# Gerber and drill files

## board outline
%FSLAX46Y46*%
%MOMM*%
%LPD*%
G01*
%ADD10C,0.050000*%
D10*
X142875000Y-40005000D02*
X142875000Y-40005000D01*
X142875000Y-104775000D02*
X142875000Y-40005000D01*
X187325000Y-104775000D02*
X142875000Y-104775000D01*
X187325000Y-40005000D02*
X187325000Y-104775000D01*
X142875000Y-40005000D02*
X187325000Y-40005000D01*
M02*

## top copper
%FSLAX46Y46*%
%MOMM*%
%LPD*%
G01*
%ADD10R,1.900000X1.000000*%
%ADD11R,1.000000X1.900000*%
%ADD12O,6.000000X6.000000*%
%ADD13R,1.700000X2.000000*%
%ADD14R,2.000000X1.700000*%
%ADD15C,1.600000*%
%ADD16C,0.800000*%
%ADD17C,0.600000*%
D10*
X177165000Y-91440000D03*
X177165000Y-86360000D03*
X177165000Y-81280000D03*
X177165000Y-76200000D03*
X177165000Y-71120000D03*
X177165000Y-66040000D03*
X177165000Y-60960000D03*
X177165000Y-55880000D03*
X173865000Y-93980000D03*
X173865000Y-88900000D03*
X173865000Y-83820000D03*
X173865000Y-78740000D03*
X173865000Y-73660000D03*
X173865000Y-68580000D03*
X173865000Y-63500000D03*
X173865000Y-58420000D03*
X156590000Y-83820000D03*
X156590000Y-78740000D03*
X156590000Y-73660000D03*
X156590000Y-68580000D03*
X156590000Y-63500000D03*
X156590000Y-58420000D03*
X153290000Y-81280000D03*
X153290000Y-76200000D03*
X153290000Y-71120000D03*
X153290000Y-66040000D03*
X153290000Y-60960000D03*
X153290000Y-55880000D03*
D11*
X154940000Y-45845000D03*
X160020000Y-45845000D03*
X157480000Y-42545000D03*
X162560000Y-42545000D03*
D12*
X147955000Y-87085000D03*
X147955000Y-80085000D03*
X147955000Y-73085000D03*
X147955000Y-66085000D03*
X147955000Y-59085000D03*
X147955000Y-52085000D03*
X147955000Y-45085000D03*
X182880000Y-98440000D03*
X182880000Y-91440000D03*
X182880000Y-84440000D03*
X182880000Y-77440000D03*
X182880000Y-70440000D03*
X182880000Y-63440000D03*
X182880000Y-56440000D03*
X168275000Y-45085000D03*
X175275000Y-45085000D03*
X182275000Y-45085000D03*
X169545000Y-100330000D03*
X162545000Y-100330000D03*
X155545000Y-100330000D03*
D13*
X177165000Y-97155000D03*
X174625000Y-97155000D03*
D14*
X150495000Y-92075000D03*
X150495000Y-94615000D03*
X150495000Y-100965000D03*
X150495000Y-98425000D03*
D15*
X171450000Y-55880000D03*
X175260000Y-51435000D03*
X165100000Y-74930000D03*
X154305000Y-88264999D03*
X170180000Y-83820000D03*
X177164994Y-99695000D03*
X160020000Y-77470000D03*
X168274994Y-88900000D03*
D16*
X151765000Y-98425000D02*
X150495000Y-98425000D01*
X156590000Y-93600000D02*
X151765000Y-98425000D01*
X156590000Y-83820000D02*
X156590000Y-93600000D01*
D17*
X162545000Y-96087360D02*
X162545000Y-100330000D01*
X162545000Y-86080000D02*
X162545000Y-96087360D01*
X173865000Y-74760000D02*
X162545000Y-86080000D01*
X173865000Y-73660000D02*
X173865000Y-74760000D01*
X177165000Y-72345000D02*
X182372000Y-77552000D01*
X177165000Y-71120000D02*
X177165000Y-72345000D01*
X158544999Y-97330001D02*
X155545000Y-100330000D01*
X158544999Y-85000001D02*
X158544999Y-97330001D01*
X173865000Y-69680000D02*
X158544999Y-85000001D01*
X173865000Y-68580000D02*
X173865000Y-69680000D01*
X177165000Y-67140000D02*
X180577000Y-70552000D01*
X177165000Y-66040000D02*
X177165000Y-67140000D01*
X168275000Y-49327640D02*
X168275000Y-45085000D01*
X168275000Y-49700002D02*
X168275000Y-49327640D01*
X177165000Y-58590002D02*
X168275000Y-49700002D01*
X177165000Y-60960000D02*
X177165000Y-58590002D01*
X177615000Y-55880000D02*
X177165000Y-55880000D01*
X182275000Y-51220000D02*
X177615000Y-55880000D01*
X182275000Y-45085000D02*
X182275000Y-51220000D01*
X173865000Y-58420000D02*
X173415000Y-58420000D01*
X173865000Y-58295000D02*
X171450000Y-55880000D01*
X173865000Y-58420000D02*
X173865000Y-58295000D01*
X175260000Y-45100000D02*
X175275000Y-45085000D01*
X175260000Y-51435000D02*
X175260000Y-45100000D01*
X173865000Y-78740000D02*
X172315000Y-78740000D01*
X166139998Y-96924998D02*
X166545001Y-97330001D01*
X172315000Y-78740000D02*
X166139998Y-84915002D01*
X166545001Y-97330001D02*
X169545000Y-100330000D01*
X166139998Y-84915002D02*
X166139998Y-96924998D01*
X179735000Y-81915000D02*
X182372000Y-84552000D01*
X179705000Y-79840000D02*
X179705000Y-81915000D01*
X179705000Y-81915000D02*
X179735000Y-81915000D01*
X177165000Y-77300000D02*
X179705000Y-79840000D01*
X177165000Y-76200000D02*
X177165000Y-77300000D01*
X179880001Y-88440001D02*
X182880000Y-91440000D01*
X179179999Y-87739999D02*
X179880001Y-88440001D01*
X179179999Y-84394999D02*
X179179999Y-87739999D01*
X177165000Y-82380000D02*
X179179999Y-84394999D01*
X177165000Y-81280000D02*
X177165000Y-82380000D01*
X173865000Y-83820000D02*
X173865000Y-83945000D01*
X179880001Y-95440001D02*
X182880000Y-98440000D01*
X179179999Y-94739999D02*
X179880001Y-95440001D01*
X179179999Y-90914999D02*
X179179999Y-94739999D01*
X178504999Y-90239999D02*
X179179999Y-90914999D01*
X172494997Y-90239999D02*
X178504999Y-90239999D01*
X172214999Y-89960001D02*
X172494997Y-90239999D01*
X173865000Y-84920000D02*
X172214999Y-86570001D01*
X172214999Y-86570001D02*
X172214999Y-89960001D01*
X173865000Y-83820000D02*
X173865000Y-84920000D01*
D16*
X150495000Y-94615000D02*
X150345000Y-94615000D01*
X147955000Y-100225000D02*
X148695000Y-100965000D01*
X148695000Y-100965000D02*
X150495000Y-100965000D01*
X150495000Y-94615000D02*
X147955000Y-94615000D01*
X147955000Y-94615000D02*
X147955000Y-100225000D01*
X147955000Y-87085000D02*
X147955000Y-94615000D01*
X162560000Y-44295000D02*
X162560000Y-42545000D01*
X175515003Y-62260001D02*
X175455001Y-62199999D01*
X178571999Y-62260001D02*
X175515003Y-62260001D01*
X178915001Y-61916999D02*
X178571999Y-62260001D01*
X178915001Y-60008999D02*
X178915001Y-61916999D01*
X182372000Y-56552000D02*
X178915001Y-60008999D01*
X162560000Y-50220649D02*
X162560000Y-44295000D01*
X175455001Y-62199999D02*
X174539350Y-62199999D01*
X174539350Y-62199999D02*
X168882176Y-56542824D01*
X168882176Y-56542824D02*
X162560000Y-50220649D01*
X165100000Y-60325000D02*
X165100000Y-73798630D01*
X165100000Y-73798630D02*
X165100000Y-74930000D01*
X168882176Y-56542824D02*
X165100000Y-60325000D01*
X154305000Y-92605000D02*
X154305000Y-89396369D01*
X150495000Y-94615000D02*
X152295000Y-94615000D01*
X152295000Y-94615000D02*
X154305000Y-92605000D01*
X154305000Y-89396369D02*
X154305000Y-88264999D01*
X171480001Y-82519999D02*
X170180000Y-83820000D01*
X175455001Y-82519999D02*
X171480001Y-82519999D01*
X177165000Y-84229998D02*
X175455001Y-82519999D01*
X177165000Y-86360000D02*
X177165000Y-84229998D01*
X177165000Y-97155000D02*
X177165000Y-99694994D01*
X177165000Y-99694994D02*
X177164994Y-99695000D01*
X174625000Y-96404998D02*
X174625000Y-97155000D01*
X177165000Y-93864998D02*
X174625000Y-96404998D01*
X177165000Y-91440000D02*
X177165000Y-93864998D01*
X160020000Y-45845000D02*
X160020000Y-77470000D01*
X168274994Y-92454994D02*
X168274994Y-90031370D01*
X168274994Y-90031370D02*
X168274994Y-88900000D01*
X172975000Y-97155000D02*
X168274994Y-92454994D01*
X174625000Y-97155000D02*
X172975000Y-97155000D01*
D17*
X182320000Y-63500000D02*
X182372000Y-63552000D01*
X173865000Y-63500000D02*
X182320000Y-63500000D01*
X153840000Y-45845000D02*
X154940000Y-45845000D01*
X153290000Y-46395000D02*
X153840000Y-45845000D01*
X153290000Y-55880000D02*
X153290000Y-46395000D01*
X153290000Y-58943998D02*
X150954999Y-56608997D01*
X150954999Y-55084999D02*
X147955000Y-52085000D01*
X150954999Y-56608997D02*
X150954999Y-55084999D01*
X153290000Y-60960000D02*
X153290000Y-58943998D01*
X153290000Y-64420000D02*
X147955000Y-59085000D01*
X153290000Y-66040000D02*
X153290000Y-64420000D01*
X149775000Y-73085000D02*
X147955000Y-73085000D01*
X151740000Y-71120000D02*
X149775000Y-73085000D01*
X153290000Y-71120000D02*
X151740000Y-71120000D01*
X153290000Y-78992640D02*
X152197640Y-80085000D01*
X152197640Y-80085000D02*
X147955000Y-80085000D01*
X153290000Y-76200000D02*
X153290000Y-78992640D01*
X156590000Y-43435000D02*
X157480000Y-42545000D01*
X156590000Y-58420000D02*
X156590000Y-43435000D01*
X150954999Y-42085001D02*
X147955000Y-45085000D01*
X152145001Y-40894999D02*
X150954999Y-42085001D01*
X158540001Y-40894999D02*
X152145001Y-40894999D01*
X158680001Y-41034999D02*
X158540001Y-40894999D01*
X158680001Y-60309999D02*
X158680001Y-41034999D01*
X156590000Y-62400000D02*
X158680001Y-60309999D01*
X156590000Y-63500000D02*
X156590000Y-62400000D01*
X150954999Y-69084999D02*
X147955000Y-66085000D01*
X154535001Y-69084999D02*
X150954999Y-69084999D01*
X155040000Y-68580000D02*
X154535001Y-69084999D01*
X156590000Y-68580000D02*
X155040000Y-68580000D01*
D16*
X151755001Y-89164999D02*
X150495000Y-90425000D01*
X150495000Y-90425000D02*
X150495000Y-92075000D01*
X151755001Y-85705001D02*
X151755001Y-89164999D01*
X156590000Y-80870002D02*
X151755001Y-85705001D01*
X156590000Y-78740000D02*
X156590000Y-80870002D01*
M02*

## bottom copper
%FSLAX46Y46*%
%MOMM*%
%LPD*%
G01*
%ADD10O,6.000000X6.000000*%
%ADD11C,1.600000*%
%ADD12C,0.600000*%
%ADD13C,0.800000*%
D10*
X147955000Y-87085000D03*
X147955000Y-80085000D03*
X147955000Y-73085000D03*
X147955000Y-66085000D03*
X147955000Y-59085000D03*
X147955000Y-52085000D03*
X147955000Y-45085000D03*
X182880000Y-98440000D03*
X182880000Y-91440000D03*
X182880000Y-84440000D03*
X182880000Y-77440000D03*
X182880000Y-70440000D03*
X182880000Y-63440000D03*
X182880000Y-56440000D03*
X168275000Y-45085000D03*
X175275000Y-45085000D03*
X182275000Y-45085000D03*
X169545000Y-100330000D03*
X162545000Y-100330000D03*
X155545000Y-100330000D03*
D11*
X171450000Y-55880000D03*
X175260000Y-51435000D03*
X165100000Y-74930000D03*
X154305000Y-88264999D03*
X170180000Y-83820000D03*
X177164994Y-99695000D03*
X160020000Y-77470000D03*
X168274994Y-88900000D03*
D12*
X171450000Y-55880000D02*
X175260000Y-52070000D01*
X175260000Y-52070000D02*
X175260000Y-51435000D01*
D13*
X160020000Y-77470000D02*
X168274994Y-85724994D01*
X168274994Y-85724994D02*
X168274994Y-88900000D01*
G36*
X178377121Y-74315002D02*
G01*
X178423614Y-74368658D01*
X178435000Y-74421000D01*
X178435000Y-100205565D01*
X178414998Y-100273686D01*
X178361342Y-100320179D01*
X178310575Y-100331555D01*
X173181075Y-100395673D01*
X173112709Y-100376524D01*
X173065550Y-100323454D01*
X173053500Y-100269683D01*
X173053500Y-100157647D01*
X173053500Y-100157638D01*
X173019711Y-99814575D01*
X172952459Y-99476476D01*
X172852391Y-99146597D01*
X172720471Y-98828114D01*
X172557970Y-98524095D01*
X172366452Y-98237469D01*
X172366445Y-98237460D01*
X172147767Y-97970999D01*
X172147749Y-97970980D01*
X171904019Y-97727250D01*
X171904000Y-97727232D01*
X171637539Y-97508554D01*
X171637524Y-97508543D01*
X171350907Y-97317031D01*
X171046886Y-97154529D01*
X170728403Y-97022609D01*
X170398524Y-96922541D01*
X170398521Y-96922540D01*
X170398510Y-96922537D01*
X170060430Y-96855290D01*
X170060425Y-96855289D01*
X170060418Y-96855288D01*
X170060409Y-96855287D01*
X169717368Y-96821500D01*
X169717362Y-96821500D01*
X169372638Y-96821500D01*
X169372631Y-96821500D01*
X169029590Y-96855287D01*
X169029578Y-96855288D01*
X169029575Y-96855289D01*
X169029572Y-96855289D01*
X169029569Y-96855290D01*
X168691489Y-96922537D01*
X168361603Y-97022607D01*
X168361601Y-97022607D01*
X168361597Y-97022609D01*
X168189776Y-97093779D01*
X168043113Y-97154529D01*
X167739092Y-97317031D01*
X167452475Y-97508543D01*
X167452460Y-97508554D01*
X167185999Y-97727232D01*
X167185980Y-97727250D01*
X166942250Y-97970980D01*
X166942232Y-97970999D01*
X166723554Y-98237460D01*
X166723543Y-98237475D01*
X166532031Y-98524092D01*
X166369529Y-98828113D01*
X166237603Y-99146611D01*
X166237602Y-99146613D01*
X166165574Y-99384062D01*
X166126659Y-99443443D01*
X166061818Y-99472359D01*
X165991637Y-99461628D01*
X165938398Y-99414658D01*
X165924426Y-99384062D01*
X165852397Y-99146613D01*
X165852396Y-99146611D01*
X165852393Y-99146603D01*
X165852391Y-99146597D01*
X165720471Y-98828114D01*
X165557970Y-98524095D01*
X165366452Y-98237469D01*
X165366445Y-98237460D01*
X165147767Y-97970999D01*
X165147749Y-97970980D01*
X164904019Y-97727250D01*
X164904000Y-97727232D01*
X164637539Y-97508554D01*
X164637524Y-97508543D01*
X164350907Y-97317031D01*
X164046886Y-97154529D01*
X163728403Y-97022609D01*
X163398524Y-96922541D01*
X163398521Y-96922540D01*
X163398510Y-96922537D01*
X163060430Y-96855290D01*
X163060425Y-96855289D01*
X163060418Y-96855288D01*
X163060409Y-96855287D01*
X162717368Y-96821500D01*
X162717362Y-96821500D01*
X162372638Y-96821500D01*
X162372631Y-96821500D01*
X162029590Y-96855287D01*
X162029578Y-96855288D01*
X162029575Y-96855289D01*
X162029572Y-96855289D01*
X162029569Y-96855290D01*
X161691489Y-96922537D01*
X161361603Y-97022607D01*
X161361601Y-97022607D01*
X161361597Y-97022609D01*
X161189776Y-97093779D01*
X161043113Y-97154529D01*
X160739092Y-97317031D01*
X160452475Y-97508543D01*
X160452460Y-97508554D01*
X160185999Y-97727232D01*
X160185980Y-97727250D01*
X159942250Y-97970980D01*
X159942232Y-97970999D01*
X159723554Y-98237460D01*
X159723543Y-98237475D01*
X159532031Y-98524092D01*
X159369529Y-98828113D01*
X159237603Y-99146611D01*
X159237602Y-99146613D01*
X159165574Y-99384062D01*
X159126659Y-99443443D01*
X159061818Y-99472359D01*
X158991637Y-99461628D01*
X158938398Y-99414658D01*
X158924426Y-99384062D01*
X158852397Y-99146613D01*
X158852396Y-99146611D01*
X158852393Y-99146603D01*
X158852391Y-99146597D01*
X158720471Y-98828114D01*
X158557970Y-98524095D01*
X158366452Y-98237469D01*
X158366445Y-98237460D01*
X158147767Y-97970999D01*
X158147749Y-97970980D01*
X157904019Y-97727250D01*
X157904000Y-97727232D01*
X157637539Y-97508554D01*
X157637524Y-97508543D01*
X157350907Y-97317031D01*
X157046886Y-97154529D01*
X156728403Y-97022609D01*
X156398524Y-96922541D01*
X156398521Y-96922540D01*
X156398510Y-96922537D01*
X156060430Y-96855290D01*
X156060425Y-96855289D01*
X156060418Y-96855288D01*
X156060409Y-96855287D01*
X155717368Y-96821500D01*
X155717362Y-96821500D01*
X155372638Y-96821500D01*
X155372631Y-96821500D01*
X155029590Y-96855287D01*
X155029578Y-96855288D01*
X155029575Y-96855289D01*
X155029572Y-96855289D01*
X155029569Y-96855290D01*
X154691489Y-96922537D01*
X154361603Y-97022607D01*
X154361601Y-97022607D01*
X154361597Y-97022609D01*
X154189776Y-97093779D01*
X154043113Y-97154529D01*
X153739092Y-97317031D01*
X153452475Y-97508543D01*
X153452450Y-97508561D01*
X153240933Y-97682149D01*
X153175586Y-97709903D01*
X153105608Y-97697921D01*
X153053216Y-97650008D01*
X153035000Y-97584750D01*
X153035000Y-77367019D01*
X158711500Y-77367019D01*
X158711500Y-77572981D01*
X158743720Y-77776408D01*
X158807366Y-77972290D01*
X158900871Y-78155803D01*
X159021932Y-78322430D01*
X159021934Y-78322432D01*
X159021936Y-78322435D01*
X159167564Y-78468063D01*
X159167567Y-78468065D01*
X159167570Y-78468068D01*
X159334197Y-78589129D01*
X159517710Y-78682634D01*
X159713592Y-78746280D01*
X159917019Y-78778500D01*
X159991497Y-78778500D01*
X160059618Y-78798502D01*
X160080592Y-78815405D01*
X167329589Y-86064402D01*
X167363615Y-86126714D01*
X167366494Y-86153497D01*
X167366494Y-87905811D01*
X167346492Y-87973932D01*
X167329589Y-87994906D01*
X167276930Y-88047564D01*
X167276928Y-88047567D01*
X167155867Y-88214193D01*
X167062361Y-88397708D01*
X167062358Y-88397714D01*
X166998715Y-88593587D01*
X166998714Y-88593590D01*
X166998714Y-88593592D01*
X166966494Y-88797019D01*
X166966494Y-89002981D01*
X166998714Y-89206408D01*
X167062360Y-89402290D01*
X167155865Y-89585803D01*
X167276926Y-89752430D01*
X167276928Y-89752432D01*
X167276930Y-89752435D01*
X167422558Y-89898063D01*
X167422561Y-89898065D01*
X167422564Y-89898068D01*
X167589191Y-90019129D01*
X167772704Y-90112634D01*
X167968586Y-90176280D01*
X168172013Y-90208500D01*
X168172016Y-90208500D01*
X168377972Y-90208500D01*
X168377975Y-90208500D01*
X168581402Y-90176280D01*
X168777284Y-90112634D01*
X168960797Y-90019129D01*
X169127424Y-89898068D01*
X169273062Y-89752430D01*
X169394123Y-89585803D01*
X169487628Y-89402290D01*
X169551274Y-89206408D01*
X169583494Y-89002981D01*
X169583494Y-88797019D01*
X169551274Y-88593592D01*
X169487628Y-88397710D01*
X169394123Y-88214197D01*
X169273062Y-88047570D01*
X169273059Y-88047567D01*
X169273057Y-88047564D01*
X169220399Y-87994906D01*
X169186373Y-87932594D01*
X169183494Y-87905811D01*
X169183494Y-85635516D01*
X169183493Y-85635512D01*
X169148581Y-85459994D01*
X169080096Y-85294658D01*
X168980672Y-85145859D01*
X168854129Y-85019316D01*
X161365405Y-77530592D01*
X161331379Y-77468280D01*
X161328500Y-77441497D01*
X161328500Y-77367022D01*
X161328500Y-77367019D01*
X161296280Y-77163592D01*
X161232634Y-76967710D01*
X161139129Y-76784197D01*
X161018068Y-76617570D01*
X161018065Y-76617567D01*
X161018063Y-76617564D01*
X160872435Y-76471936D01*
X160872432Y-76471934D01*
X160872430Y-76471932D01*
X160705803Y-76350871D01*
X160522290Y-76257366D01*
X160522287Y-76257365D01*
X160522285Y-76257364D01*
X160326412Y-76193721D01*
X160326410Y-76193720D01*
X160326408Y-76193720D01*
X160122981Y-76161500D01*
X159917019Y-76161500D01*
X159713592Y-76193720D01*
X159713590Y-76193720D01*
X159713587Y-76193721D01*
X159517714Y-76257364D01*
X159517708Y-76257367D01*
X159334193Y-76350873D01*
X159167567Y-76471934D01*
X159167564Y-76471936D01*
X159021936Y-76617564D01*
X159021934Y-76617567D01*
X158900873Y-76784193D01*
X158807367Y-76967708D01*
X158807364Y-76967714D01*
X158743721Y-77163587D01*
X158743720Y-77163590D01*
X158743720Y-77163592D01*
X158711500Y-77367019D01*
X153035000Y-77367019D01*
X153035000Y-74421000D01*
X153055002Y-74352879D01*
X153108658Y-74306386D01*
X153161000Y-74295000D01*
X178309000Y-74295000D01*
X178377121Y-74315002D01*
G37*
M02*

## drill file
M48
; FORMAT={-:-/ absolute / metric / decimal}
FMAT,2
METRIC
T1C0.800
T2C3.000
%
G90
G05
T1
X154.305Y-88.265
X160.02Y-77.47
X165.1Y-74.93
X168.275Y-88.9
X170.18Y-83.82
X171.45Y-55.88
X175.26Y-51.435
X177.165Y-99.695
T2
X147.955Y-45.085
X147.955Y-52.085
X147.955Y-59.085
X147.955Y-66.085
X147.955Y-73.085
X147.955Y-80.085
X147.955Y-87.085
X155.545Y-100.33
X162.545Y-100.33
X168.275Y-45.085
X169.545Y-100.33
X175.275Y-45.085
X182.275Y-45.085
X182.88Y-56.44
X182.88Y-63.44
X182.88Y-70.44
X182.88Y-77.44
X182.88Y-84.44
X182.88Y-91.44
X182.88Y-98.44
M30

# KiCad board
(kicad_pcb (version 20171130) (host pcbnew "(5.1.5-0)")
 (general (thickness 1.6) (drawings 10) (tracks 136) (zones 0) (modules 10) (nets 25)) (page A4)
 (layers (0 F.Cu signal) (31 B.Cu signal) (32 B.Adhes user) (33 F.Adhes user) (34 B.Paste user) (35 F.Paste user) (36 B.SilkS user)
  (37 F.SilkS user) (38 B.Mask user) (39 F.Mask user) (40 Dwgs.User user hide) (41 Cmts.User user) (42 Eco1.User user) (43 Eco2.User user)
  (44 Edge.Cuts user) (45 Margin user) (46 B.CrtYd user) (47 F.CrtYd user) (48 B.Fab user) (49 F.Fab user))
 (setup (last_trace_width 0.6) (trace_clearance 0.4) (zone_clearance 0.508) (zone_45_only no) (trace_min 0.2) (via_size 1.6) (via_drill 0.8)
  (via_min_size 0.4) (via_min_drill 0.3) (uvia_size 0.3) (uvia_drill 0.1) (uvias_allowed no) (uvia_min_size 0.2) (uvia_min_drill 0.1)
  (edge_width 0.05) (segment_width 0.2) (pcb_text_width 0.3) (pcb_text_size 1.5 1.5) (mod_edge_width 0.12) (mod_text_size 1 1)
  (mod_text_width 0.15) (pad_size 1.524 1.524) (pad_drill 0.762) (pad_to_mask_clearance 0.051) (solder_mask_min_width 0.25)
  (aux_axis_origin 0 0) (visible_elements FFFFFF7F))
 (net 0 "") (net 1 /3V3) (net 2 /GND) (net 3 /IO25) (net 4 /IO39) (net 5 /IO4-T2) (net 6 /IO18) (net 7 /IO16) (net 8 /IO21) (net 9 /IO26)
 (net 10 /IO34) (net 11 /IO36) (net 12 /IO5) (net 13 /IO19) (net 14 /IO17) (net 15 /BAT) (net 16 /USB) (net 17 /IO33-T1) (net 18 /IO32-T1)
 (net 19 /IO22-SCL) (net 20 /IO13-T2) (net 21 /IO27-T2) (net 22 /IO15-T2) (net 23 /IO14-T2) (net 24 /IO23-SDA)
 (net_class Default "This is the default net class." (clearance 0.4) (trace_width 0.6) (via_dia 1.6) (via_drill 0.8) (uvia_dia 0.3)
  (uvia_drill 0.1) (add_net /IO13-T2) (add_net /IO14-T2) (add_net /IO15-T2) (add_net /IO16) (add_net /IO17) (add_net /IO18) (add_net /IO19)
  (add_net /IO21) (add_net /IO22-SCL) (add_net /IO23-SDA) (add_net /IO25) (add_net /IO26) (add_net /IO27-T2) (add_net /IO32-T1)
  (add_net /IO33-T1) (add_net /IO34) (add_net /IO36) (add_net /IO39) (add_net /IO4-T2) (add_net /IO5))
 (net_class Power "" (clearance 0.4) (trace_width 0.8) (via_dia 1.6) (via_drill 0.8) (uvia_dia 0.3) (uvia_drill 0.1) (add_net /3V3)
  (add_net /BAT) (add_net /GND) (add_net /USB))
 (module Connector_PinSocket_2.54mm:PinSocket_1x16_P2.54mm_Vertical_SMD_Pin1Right (layer F.Cu) (at 175.515 74.93)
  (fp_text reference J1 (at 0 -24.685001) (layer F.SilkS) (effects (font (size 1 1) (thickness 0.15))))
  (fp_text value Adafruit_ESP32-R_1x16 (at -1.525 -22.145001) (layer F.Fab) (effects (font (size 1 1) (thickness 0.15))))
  (pad 15 smd rect (at 1.65 16.51) (size 1.9 1) (layers F.Cu F.Paste F.Mask) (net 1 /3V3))
  (pad 13 smd rect (at 1.65 11.43) (size 1.9 1) (layers F.Cu F.Paste F.Mask) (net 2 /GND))
  (pad 11 smd rect (at 1.65 6.35) (size 1.9 1) (layers F.Cu F.Paste F.Mask) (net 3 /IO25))
  (pad 9 smd rect (at 1.65 1.27) (size 1.9 1) (layers F.Cu F.Paste F.Mask) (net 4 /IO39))
  (pad 7 smd rect (at 1.65 -3.81) (size 1.9 1) (layers F.Cu F.Paste F.Mask) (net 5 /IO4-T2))
  (pad 5 smd rect (at 1.65 -8.89) (size 1.9 1) (layers F.Cu F.Paste F.Mask) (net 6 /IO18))
  (pad 3 smd rect (at 1.65 -13.97) (size 1.9 1) (layers F.Cu F.Paste F.Mask) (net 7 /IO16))
  (pad 1 smd rect (at 1.65 -19.05) (size 1.9 1) (layers F.Cu F.Paste F.Mask) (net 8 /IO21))
  (pad 16 smd rect (at -1.65 19.05) (size 1.9 1) (layers F.Cu F.Paste F.Mask))
  (pad 14 smd rect (at -1.65 13.97) (size 1.9 1) (layers F.Cu F.Paste F.Mask))
  (pad 12 smd rect (at -1.65 8.89) (size 1.9 1) (layers F.Cu F.Paste F.Mask) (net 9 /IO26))
  (pad 10 smd rect (at -1.65 3.81) (size 1.9 1) (layers F.Cu F.Paste F.Mask) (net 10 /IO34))
  (pad 8 smd rect (at -1.65 -1.27) (size 1.9 1) (layers F.Cu F.Paste F.Mask) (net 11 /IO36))
  (pad 6 smd rect (at -1.65 -6.35) (size 1.9 1) (layers F.Cu F.Paste F.Mask) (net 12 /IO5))
  (pad 4 smd rect (at -1.65 -11.43) (size 1.9 1) (layers F.Cu F.Paste F.Mask) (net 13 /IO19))
  (pad 2 smd rect (at -1.65 -16.51) (size 1.9 1) (layers F.Cu F.Paste F.Mask) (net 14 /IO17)))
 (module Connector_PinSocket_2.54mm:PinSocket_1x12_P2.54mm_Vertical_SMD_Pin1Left (layer F.Cu) (at 154.94 69.85)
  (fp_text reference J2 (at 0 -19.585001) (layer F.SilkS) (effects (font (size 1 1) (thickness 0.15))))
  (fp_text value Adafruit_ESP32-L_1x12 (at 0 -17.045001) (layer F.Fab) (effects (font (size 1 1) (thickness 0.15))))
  (pad 12 smd rect (at 1.65 13.97) (size 1.9 1) (layers F.Cu F.Paste F.Mask) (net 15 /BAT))
  (pad 10 smd rect (at 1.65 8.89) (size 1.9 1) (layers F.Cu F.Paste F.Mask) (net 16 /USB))
  (pad 8 smd rect (at 1.65 3.81) (size 1.9 1) (layers F.Cu F.Paste F.Mask))
  (pad 6 smd rect (at 1.65 -1.27) (size 1.9 1) (layers F.Cu F.Paste F.Mask) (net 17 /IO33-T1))
  (pad 4 smd rect (at 1.65 -6.35) (size 1.9 1) (layers F.Cu F.Paste F.Mask) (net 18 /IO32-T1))
  (pad 2 smd rect (at 1.65 -11.43) (size 1.9 1) (layers F.Cu F.Paste F.Mask) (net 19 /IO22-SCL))
  (pad 11 smd rect (at -1.65 11.43) (size 1.9 1) (layers F.Cu F.Paste F.Mask))
  (pad 9 smd rect (at -1.65 6.35) (size 1.9 1) (layers F.Cu F.Paste F.Mask) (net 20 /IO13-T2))
  (pad 7 smd rect (at -1.65 1.27) (size 1.9 1) (layers F.Cu F.Paste F.Mask) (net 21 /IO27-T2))
  (pad 5 smd rect (at -1.65 -3.81) (size 1.9 1) (layers F.Cu F.Paste F.Mask) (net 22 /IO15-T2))
  (pad 3 smd rect (at -1.65 -8.89) (size 1.9 1) (layers F.Cu F.Paste F.Mask) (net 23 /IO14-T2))
  (pad 1 smd rect (at -1.65 -13.97) (size 1.9 1) (layers F.Cu F.Paste F.Mask) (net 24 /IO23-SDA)))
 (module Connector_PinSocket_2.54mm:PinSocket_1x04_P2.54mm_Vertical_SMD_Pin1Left (layer F.Cu) (at 158.75 44.195 270)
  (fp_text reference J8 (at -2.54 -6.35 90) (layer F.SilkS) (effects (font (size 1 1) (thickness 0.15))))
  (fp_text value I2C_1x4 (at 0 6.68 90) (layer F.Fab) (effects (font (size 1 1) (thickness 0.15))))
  (pad 4 smd rect (at 1.65 3.81 270) (size 1.9 1) (layers F.Cu F.Paste F.Mask) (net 24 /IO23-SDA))
  (pad 2 smd rect (at 1.65 -1.27 270) (size 1.9 1) (layers F.Cu F.Paste F.Mask) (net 1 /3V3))
  (pad 3 smd rect (at -1.65 1.27 270) (size 1.9 1) (layers F.Cu F.Paste F.Mask) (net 19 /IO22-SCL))
  (pad 1 smd rect (at -1.65 -3.81 270) (size 1.9 1) (layers F.Cu F.Paste F.Mask) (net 2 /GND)))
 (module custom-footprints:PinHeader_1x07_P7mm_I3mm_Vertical (layer F.Cu) (at 147.955 45.085)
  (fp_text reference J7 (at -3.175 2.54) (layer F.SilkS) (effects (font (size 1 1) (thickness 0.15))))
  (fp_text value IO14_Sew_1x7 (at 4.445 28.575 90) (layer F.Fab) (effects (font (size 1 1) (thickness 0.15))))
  (pad 7 thru_hole oval (at 0 42) (size 6 6) (drill 3) (layers *.Cu *.Mask) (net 2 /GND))
  (pad 6 thru_hole oval (at 0 35) (size 6 6) (drill 3) (layers *.Cu *.Mask) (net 20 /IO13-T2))
  (pad 5 thru_hole oval (at 0 28) (size 6 6) (drill 3) (layers *.Cu *.Mask) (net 21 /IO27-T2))
  (pad 4 thru_hole oval (at 0 21) (size 6 6) (drill 3) (layers *.Cu *.Mask) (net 17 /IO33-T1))
  (pad 3 thru_hole oval (at 0 14) (size 6 6) (drill 3) (layers *.Cu *.Mask) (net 22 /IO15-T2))
  (pad 2 thru_hole oval (at 0 7) (size 6 6) (drill 3) (layers *.Cu *.Mask) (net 23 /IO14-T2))
  (pad 1 thru_hole oval (at 0 0) (size 6 6) (drill 3) (layers *.Cu *.Mask) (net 18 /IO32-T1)))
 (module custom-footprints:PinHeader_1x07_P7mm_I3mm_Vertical (layer F.Cu) (at 182.88 56.44)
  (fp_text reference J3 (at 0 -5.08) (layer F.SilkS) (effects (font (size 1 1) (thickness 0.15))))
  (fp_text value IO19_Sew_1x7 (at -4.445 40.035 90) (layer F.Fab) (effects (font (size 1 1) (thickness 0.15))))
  (pad 7 thru_hole oval (at 0 42) (size 6 6) (drill 3) (layers *.Cu *.Mask) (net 9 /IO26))
  (pad 6 thru_hole oval (at 0 35) (size 6 6) (drill 3) (layers *.Cu *.Mask) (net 3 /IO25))
  (pad 5 thru_hole oval (at 0 28) (size 6 6) (drill 3) (layers *.Cu *.Mask) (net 4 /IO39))
  (pad 4 thru_hole oval (at 0 21) (size 6 6) (drill 3) (layers *.Cu *.Mask) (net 5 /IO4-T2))
  (pad 3 thru_hole oval (at 0 14) (size 6 6) (drill 3) (layers *.Cu *.Mask) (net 6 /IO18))
  (pad 2 thru_hole oval (at 0 7) (size 6 6) (drill 3) (layers *.Cu *.Mask) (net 13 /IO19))
  (pad 1 thru_hole oval (at 0 0) (size 6 6) (drill 3) (layers *.Cu *.Mask) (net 2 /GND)))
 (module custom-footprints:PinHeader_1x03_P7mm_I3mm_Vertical (layer F.Cu) (at 182.275 45.085 270)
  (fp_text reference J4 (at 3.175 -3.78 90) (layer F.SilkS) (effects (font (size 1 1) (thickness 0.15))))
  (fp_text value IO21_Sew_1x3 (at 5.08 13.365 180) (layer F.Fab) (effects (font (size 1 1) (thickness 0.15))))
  (pad 3 thru_hole oval (at 0 14 270) (size 6 6) (drill 3) (layers *.Cu *.Mask) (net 7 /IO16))
  (pad 2 thru_hole oval (at 0 7 270) (size 6 6) (drill 3) (layers *.Cu *.Mask) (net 14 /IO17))
  (pad 1 thru_hole oval (at 0 0 270) (size 6 6) (drill 3) (layers *.Cu *.Mask) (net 8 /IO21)))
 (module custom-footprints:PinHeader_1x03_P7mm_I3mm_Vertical (layer F.Cu) (at 155.545 100.33 90)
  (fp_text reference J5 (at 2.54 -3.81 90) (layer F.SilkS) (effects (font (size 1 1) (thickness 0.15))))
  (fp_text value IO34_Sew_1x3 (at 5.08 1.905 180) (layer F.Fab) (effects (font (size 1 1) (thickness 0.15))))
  (pad 3 thru_hole oval (at 0 14 90) (size 6 6) (drill 3) (layers *.Cu *.Mask) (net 10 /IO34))
  (pad 2 thru_hole oval (at 0 7 90) (size 6 6) (drill 3) (layers *.Cu *.Mask) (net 11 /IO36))
  (pad 1 thru_hole oval (at 0 0 90) (size 6 6) (drill 3) (layers *.Cu *.Mask) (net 12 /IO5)))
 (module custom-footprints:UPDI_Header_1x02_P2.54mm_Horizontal (layer F.Cu) (at 177.165 97.155 270)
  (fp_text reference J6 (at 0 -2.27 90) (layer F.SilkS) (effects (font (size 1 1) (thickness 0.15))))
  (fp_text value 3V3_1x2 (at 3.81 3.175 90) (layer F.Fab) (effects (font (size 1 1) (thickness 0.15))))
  (pad 2 smd rect (at 0 0 270) (size 2 1.7) (layers F.Cu F.Paste F.Mask) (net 2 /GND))
  (pad 1 smd rect (at 0 2.54 270) (size 2 1.7) (layers F.Cu F.Paste F.Mask) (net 1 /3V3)))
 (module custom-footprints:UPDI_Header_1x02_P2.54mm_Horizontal (layer F.Cu) (at 150.495 94.615 180)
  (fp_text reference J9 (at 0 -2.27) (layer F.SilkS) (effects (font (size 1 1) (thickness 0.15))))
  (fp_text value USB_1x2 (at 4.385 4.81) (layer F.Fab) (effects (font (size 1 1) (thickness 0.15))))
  (pad 1 smd rect (at 0 2.54 180) (size 2 1.7) (layers F.Cu F.Paste F.Mask) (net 16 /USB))
  (pad 2 smd rect (at 0 0 180) (size 2 1.7) (layers F.Cu F.Paste F.Mask) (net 2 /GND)))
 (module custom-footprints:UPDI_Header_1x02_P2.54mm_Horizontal (layer F.Cu) (at 150.495 100.965 180)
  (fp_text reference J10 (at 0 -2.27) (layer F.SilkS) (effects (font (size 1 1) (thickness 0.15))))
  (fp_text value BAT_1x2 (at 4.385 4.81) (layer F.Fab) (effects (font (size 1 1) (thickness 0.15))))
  (pad 2 smd rect (at 0 0 180) (size 2 1.7) (layers F.Cu F.Paste F.Mask) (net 2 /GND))
  (pad 1 smd rect (at 0 2.54 180) (size 2 1.7) (layers F.Cu F.Paste F.Mask) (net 15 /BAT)))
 (gr_line (start 142.875 40.005) (end 142.875 40.005) (layer Edge.Cuts) (width 0.05))
 (gr_line (start 142.875 104.775) (end 142.875 40.005) (layer Edge.Cuts) (width 0.05))
 (gr_line (start 187.325 104.775) (end 142.875 104.775) (layer Edge.Cuts) (width 0.05))
 (gr_line (start 187.325 40.005) (end 187.325 104.775) (layer Edge.Cuts) (width 0.05))
 (gr_line (start 142.875 40.005) (end 187.325 40.005) (layer Edge.Cuts) (width 0.05))
 (segment (start 151.765 98.425) (end 150.495 98.425) (width 0.8) (layer F.Cu) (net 15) (status 20))
 (segment (start 156.59 93.6) (end 151.765 98.425) (width 0.8) (layer F.Cu) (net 15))
 (segment (start 156.59 83.82) (end 156.59 93.6) (width 0.8) (layer F.Cu) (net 15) (status 10))
 (segment (start 162.545 96.08736) (end 162.545 100.33) (width 0.6) (layer F.Cu) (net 11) (status 20))
 (segment (start 162.545 86.08) (end 162.545 96.08736) (width 0.6) (layer F.Cu) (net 11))
 (segment (start 173.865 74.76) (end 162.545 86.08) (width 0.6) (layer F.Cu) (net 11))
 (segment (start 173.865 73.66) (end 173.865 74.76) (width 0.6) (layer F.Cu) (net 11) (status 10))
 (segment (start 177.165 72.345) (end 182.372 77.552) (width 0.6) (layer F.Cu) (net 5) (status 20))
 (segment (start 177.165 71.12) (end 177.165 72.345) (width 0.6) (layer F.Cu) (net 5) (status 10))
 (segment (start 158.544999 97.330001) (end 155.545 100.33) (width 0.6) (layer F.Cu) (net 12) (status 20))
 (segment (start 158.544999 85.000001) (end 158.544999 97.330001) (width 0.6) (layer F.Cu) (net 12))
 (segment (start 173.865 69.68) (end 158.544999 85.000001) (width 0.6) (layer F.Cu) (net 12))
 (segment (start 173.865 68.58) (end 173.865 69.68) (width 0.6) (layer F.Cu) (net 12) (status 10))
 (segment (start 177.165 67.14) (end 180.577 70.552) (width 0.6) (layer F.Cu) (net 6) (status 20))
 (segment (start 177.165 66.04) (end 177.165 67.14) (width 0.6) (layer F.Cu) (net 6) (status 10))
 (segment (start 168.275 49.32764) (end 168.275 45.085) (width 0.6) (layer F.Cu) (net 7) (status 20))
 (segment (start 168.275 49.700002) (end 168.275 49.32764) (width 0.6) (layer F.Cu) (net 7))
 (segment (start 177.165 58.590002) (end 168.275 49.700002) (width 0.6) (layer F.Cu) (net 7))
 (segment (start 177.165 60.96) (end 177.165 58.590002) (width 0.6) (layer F.Cu) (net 7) (status 10))
 (segment (start 177.615 55.88) (end 177.165 55.88) (width 0.6) (layer F.Cu) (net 8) (status 30))
 (segment (start 182.275 51.22) (end 177.615 55.88) (width 0.6) (layer F.Cu) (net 8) (status 20))
 (segment (start 182.275 45.085) (end 182.275 51.22) (width 0.6) (layer F.Cu) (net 8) (status 10))
 (segment (start 173.865 58.42) (end 173.415 58.42) (width 0.6) (layer F.Cu) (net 14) (status 30))
 (segment (start 173.865 58.295) (end 171.45 55.88) (width 0.6) (layer F.Cu) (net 14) (status 10))
 (via (at 171.45 55.88) (size 1.6) (drill 0.8) (layers F.Cu B.Cu) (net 14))
 (segment (start 173.865 58.42) (end 173.865 58.295) (width 0.6) (layer F.Cu) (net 14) (status 30))
 (segment (start 171.45 55.88) (end 175.26 52.07) (width 0.6) (layer B.Cu) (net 14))
 (via (at 175.26 51.435) (size 1.6) (drill 0.8) (layers F.Cu B.Cu) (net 14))
 (segment (start 175.26 52.07) (end 175.26 51.435) (width 0.6) (layer B.Cu) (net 14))
 (segment (start 175.26 45.1) (end 175.275 45.085) (width 0.6) (layer F.Cu) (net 14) (status 30))
 (segment (start 175.26 51.435) (end 175.26 45.1) (width 0.6) (layer F.Cu) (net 14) (status 20))
 (segment (start 173.865 78.74) (end 172.315 78.74) (width 0.6) (layer F.Cu) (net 10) (status 10))
 (segment (start 166.139998 96.924998) (end 166.545001 97.330001) (width 0.6) (layer F.Cu) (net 10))
 (segment (start 172.315 78.74) (end 166.139998 84.915002) (width 0.6) (layer F.Cu) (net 10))
 (segment (start 166.545001 97.330001) (end 169.545 100.33) (width 0.6) (layer F.Cu) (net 10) (status 20))
 (segment (start 166.139998 84.915002) (end 166.139998 96.924998) (width 0.6) (layer F.Cu) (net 10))
 (segment (start 179.735 81.915) (end 182.372 84.552) (width 0.6) (layer F.Cu) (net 4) (status 20))
 (segment (start 179.705 79.84) (end 179.705 81.915) (width 0.6) (layer F.Cu) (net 4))
 (segment (start 179.705 81.915) (end 179.735 81.915) (width 0.6) (layer F.Cu) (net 4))
 (segment (start 177.165 77.3) (end 179.705 79.84) (width 0.6) (layer F.Cu) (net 4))
 (segment (start 177.165 76.2) (end 177.165 77.3) (width 0.6) (layer F.Cu) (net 4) (status 10))
 (segment (start 179.880001 88.440001) (end 182.88 91.44) (width 0.6) (layer F.Cu) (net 3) (status 20))
 (segment (start 179.179999 87.739999) (end 179.880001 88.440001) (width 0.6) (layer F.Cu) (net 3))
 (segment (start 179.179999 84.394999) (end 179.179999 87.739999) (width 0.6) (layer F.Cu) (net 3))
 (segment (start 177.165 82.38) (end 179.179999 84.394999) (width 0.6) (layer F.Cu) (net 3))
 (segment (start 177.165 81.28) (end 177.165 82.38) (width 0.6) (layer F.Cu) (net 3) (status 10))
 (segment (start 173.865 83.82) (end 173.865 83.945) (width 0.6) (layer F.Cu) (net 9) (status 30))
 (segment (start 179.880001 95.440001) (end 182.88 98.44) (width 0.6) (layer F.Cu) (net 9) (status 20))
 (segment (start 179.179999 94.739999) (end 179.880001 95.440001) (width 0.6) (layer F.Cu) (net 9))
 (segment (start 179.179999 90.914999) (end 179.179999 94.739999) (width 0.6) (layer F.Cu) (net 9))
 (segment (start 178.504999 90.239999) (end 179.179999 90.914999) (width 0.6) (layer F.Cu) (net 9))
 (segment (start 172.494997 90.239999) (end 178.504999 90.239999) (width 0.6) (layer F.Cu) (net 9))
 (segment (start 172.214999 89.960001) (end 172.494997 90.239999) (width 0.6) (layer F.Cu) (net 9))
 (segment (start 173.865 84.92) (end 172.214999 86.570001) (width 0.6) (layer F.Cu) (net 9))
 (segment (start 172.214999 86.570001) (end 172.214999 89.960001) (width 0.6) (layer F.Cu) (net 9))
 (segment (start 173.865 83.82) (end 173.865 84.92) (width 0.6) (layer F.Cu) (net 9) (status 10))
 (segment (start 150.495 94.615) (end 150.345 94.615) (width 0.8) (layer F.Cu) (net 2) (status 30))
 (segment (start 147.955 100.225) (end 148.695 100.965) (width 0.8) (layer F.Cu) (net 2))
 (segment (start 148.695 100.965) (end 150.495 100.965) (width 0.8) (layer F.Cu) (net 2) (status 20))
 (segment (start 150.495 94.615) (end 147.955 94.615) (width 0.8) (layer F.Cu) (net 2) (status 10))
 (segment (start 147.955 94.615) (end 147.955 100.225) (width 0.8) (layer F.Cu) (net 2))
 (segment (start 147.955 87.085) (end 147.955 94.615) (width 0.8) (layer F.Cu) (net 2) (status 10))
 (segment (start 162.56 44.295) (end 162.56 42.545) (width 0.8) (layer F.Cu) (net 2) (status 20))
 (segment (start 175.515003 62.260001) (end 175.455001 62.199999) (width 0.8) (layer F.Cu) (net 2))
 (segment (start 178.571999 62.260001) (end 175.515003 62.260001) (width 0.8) (layer F.Cu) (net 2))
 (segment (start 178.915001 61.916999) (end 178.571999 62.260001) (width 0.8) (layer F.Cu) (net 2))
 (segment (start 178.915001 60.008999) (end 178.915001 61.916999) (width 0.8) (layer F.Cu) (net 2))
 (segment (start 182.372 56.552) (end 178.915001 60.008999) (width 0.8) (layer F.Cu) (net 2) (status 10))
 (segment (start 162.56 50.220649) (end 162.56 44.295) (width 0.8) (layer F.Cu) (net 2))
 (segment (start 175.455001 62.199999) (end 174.53935 62.199999) (width 0.8) (layer F.Cu) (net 2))
 (segment (start 174.53935 62.199999) (end 168.882176 56.542824) (width 0.8) (layer F.Cu) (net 2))
 (segment (start 168.882176 56.542824) (end 162.56 50.220649) (width 0.8) (layer F.Cu) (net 2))
 (segment (start 165.1 60.325) (end 165.1 73.79863) (width 0.8) (layer F.Cu) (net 2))
 (segment (start 165.1 73.79863) (end 165.1 74.93) (width 0.8) (layer F.Cu) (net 2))
 (segment (start 168.882176 56.542824) (end 165.1 60.325) (width 0.8) (layer F.Cu) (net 2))
 (via (at 165.1 74.93) (size 1.6) (drill 0.8) (layers F.Cu B.Cu) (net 2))
 (via (at 154.305 88.264999) (size 1.6) (drill 0.8) (layers F.Cu B.Cu) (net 2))
 (segment (start 154.305 92.605) (end 154.305 89.396369) (width 0.8) (layer F.Cu) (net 2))
 (segment (start 150.495 94.615) (end 152.295 94.615) (width 0.8) (layer F.Cu) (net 2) (status 10))
 (segment (start 152.295 94.615) (end 154.305 92.605) (width 0.8) (layer F.Cu) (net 2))
 (segment (start 154.305 89.396369) (end 154.305 88.264999) (width 0.8) (layer F.Cu) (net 2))
 (via (at 170.18 83.82) (size 1.6) (drill 0.8) (layers F.Cu B.Cu) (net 2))
 (segment (start 171.480001 82.519999) (end 170.18 83.82) (width 0.8) (layer F.Cu) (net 2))
 (segment (start 175.455001 82.519999) (end 171.480001 82.519999) (width 0.8) (layer F.Cu) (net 2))
 (segment (start 177.165 84.229998) (end 175.455001 82.519999) (width 0.8) (layer F.Cu) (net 2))
 (segment (start 177.165 86.36) (end 177.165 84.229998) (width 0.8) (layer F.Cu) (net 2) (status 10))
 (via (at 177.164994 99.695) (size 1.6) (drill 0.8) (layers F.Cu B.Cu) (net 2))
 (segment (start 177.165 97.155) (end 177.165 99.694994) (width 0.8) (layer F.Cu) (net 2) (status 10))
 (segment (start 177.165 99.694994) (end 177.164994 99.695) (width 0.8) (layer F.Cu) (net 2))
 (segment (start 174.625 96.404998) (end 174.625 97.155) (width 0.8) (layer F.Cu) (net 1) (status 30))
 (segment (start 177.165 93.864998) (end 174.625 96.404998) (width 0.8) (layer F.Cu) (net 1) (status 20))
 (segment (start 177.165 91.44) (end 177.165 93.864998) (width 0.8) (layer F.Cu) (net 1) (status 10))
 (segment (start 160.02 45.845) (end 160.02 77.47) (width 0.8) (layer F.Cu) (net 1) (status 10))
 (via (at 160.02 77.47) (size 1.6) (drill 0.8) (layers F.Cu B.Cu) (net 1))
 (via (at 168.274994 88.9) (size 1.6) (drill 0.8) (layers F.Cu B.Cu) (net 1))
 (segment (start 160.02 77.47) (end 168.274994 85.724994) (width 0.8) (layer B.Cu) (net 1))
 (segment (start 168.274994 85.724994) (end 168.274994 88.9) (width 0.8) (layer B.Cu) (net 1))
 (segment (start 168.274994 92.454994) (end 168.274994 90.03137) (width 0.8) (layer F.Cu) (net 1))
 (segment (start 168.274994 90.03137) (end 168.274994 88.9) (width 0.8) (layer F.Cu) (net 1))
 (segment (start 172.975 97.155) (end 168.274994 92.454994) (width 0.8) (layer F.Cu) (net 1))
 (segment (start 174.625 97.155) (end 172.975 97.155) (width 0.8) (layer F.Cu) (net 1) (status 10))
 (segment (start 182.32 63.5) (end 182.372 63.552) (width 0.6) (layer F.Cu) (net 13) (status 30))
 (segment (start 173.865 63.5) (end 182.32 63.5) (width 0.6) (layer F.Cu) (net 13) (status 30))
 (segment (start 153.84 45.845) (end 154.94 45.845) (width 0.6) (layer F.Cu) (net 24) (status 20))
 (segment (start 153.29 46.395) (end 153.84 45.845) (width 0.6) (layer F.Cu) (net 24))
 (segment (start 153.29 55.88) (end 153.29 46.395) (width 0.6) (layer F.Cu) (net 24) (status 10))
 (segment (start 153.29 58.943998) (end 150.954999 56.608997) (width 0.6) (layer F.Cu) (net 23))
 (segment (start 150.954999 55.084999) (end 147.955 52.085) (width 0.6) (layer F.Cu) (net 23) (status 20))
 (segment (start 150.954999 56.608997) (end 150.954999 55.084999) (width 0.6) (layer F.Cu) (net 23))
 (segment (start 153.29 60.96) (end 153.29 58.943998) (width 0.6) (layer F.Cu) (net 23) (status 10))
 (segment (start 153.29 64.42) (end 147.955 59.085) (width 0.6) (layer F.Cu) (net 22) (status 20))
 (segment (start 153.29 66.04) (end 153.29 64.42) (width 0.6) (layer F.Cu) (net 22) (status 10))
 (segment (start 149.775 73.085) (end 147.955 73.085) (width 0.6) (layer F.Cu) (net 21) (status 30))
 (segment (start 151.74 71.12) (end 149.775 73.085) (width 0.6) (layer F.Cu) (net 21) (status 20))
 (segment (start 153.29 71.12) (end 151.74 71.12) (width 0.6) (layer F.Cu) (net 21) (status 10))
 (segment (start 153.29 78.99264) (end 152.19764 80.085) (width 0.6) (layer F.Cu) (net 20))
 (segment (start 152.19764 80.085) (end 147.955 80.085) (width 0.6) (layer F.Cu) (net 20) (status 20))
 (segment (start 153.29 76.2) (end 153.29 78.99264) (width 0.6) (layer F.Cu) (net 20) (status 10))
 (segment (start 156.59 43.435) (end 157.48 42.545) (width 0.6) (layer F.Cu) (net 19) (status 20))
 (segment (start 156.59 58.42) (end 156.59 43.435) (width 0.6) (layer F.Cu) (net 19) (status 10))
 (segment (start 150.954999 42.085001) (end 147.955 45.085) (width 0.6) (layer F.Cu) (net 18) (status 20))
 (segment (start 152.145001 40.894999) (end 150.954999 42.085001) (width 0.6) (layer F.Cu) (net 18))
 (segment (start 158.540001 40.894999) (end 152.145001 40.894999) (width 0.6) (layer F.Cu) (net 18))
 (segment (start 158.680001 41.034999) (end 158.540001 40.894999) (width 0.6) (layer F.Cu) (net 18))
 (segment (start 158.680001 60.309999) (end 158.680001 41.034999) (width 0.6) (layer F.Cu) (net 18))
 (segment (start 156.59 62.4) (end 158.680001 60.309999) (width 0.6) (layer F.Cu) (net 18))
 (segment (start 156.59 63.5) (end 156.59 62.4) (width 0.6) (layer F.Cu) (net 18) (status 10))
 (segment (start 150.954999 69.084999) (end 147.955 66.085) (width 0.6) (layer F.Cu) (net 17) (status 20))
 (segment (start 154.535001 69.084999) (end 150.954999 69.084999) (width 0.6) (layer F.Cu) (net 17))
 (segment (start 155.04 68.58) (end 154.535001 69.084999) (width 0.6) (layer F.Cu) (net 17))
 (segment (start 156.59 68.58) (end 155.04 68.58) (width 0.6) (layer F.Cu) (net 17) (status 10))
 (segment (start 151.755001 89.164999) (end 150.495 90.425) (width 0.8) (layer F.Cu) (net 16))
 (segment (start 150.495 90.425) (end 150.495 92.075) (width 0.8) (layer F.Cu) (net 16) (status 20))
 (segment (start 151.755001 85.705001) (end 151.755001 89.164999) (width 0.8) (layer F.Cu) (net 16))
 (segment (start 156.59 80.870002) (end 151.755001 85.705001) (width 0.8) (layer F.Cu) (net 16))
 (segment (start 156.59 78.74) (end 156.59 80.870002) (width 0.8) (layer F.Cu) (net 16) (status 10))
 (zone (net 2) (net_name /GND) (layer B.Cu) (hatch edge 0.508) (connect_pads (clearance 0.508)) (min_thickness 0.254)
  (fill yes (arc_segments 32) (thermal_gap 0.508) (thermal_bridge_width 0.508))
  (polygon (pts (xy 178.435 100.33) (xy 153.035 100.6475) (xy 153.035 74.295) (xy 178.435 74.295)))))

